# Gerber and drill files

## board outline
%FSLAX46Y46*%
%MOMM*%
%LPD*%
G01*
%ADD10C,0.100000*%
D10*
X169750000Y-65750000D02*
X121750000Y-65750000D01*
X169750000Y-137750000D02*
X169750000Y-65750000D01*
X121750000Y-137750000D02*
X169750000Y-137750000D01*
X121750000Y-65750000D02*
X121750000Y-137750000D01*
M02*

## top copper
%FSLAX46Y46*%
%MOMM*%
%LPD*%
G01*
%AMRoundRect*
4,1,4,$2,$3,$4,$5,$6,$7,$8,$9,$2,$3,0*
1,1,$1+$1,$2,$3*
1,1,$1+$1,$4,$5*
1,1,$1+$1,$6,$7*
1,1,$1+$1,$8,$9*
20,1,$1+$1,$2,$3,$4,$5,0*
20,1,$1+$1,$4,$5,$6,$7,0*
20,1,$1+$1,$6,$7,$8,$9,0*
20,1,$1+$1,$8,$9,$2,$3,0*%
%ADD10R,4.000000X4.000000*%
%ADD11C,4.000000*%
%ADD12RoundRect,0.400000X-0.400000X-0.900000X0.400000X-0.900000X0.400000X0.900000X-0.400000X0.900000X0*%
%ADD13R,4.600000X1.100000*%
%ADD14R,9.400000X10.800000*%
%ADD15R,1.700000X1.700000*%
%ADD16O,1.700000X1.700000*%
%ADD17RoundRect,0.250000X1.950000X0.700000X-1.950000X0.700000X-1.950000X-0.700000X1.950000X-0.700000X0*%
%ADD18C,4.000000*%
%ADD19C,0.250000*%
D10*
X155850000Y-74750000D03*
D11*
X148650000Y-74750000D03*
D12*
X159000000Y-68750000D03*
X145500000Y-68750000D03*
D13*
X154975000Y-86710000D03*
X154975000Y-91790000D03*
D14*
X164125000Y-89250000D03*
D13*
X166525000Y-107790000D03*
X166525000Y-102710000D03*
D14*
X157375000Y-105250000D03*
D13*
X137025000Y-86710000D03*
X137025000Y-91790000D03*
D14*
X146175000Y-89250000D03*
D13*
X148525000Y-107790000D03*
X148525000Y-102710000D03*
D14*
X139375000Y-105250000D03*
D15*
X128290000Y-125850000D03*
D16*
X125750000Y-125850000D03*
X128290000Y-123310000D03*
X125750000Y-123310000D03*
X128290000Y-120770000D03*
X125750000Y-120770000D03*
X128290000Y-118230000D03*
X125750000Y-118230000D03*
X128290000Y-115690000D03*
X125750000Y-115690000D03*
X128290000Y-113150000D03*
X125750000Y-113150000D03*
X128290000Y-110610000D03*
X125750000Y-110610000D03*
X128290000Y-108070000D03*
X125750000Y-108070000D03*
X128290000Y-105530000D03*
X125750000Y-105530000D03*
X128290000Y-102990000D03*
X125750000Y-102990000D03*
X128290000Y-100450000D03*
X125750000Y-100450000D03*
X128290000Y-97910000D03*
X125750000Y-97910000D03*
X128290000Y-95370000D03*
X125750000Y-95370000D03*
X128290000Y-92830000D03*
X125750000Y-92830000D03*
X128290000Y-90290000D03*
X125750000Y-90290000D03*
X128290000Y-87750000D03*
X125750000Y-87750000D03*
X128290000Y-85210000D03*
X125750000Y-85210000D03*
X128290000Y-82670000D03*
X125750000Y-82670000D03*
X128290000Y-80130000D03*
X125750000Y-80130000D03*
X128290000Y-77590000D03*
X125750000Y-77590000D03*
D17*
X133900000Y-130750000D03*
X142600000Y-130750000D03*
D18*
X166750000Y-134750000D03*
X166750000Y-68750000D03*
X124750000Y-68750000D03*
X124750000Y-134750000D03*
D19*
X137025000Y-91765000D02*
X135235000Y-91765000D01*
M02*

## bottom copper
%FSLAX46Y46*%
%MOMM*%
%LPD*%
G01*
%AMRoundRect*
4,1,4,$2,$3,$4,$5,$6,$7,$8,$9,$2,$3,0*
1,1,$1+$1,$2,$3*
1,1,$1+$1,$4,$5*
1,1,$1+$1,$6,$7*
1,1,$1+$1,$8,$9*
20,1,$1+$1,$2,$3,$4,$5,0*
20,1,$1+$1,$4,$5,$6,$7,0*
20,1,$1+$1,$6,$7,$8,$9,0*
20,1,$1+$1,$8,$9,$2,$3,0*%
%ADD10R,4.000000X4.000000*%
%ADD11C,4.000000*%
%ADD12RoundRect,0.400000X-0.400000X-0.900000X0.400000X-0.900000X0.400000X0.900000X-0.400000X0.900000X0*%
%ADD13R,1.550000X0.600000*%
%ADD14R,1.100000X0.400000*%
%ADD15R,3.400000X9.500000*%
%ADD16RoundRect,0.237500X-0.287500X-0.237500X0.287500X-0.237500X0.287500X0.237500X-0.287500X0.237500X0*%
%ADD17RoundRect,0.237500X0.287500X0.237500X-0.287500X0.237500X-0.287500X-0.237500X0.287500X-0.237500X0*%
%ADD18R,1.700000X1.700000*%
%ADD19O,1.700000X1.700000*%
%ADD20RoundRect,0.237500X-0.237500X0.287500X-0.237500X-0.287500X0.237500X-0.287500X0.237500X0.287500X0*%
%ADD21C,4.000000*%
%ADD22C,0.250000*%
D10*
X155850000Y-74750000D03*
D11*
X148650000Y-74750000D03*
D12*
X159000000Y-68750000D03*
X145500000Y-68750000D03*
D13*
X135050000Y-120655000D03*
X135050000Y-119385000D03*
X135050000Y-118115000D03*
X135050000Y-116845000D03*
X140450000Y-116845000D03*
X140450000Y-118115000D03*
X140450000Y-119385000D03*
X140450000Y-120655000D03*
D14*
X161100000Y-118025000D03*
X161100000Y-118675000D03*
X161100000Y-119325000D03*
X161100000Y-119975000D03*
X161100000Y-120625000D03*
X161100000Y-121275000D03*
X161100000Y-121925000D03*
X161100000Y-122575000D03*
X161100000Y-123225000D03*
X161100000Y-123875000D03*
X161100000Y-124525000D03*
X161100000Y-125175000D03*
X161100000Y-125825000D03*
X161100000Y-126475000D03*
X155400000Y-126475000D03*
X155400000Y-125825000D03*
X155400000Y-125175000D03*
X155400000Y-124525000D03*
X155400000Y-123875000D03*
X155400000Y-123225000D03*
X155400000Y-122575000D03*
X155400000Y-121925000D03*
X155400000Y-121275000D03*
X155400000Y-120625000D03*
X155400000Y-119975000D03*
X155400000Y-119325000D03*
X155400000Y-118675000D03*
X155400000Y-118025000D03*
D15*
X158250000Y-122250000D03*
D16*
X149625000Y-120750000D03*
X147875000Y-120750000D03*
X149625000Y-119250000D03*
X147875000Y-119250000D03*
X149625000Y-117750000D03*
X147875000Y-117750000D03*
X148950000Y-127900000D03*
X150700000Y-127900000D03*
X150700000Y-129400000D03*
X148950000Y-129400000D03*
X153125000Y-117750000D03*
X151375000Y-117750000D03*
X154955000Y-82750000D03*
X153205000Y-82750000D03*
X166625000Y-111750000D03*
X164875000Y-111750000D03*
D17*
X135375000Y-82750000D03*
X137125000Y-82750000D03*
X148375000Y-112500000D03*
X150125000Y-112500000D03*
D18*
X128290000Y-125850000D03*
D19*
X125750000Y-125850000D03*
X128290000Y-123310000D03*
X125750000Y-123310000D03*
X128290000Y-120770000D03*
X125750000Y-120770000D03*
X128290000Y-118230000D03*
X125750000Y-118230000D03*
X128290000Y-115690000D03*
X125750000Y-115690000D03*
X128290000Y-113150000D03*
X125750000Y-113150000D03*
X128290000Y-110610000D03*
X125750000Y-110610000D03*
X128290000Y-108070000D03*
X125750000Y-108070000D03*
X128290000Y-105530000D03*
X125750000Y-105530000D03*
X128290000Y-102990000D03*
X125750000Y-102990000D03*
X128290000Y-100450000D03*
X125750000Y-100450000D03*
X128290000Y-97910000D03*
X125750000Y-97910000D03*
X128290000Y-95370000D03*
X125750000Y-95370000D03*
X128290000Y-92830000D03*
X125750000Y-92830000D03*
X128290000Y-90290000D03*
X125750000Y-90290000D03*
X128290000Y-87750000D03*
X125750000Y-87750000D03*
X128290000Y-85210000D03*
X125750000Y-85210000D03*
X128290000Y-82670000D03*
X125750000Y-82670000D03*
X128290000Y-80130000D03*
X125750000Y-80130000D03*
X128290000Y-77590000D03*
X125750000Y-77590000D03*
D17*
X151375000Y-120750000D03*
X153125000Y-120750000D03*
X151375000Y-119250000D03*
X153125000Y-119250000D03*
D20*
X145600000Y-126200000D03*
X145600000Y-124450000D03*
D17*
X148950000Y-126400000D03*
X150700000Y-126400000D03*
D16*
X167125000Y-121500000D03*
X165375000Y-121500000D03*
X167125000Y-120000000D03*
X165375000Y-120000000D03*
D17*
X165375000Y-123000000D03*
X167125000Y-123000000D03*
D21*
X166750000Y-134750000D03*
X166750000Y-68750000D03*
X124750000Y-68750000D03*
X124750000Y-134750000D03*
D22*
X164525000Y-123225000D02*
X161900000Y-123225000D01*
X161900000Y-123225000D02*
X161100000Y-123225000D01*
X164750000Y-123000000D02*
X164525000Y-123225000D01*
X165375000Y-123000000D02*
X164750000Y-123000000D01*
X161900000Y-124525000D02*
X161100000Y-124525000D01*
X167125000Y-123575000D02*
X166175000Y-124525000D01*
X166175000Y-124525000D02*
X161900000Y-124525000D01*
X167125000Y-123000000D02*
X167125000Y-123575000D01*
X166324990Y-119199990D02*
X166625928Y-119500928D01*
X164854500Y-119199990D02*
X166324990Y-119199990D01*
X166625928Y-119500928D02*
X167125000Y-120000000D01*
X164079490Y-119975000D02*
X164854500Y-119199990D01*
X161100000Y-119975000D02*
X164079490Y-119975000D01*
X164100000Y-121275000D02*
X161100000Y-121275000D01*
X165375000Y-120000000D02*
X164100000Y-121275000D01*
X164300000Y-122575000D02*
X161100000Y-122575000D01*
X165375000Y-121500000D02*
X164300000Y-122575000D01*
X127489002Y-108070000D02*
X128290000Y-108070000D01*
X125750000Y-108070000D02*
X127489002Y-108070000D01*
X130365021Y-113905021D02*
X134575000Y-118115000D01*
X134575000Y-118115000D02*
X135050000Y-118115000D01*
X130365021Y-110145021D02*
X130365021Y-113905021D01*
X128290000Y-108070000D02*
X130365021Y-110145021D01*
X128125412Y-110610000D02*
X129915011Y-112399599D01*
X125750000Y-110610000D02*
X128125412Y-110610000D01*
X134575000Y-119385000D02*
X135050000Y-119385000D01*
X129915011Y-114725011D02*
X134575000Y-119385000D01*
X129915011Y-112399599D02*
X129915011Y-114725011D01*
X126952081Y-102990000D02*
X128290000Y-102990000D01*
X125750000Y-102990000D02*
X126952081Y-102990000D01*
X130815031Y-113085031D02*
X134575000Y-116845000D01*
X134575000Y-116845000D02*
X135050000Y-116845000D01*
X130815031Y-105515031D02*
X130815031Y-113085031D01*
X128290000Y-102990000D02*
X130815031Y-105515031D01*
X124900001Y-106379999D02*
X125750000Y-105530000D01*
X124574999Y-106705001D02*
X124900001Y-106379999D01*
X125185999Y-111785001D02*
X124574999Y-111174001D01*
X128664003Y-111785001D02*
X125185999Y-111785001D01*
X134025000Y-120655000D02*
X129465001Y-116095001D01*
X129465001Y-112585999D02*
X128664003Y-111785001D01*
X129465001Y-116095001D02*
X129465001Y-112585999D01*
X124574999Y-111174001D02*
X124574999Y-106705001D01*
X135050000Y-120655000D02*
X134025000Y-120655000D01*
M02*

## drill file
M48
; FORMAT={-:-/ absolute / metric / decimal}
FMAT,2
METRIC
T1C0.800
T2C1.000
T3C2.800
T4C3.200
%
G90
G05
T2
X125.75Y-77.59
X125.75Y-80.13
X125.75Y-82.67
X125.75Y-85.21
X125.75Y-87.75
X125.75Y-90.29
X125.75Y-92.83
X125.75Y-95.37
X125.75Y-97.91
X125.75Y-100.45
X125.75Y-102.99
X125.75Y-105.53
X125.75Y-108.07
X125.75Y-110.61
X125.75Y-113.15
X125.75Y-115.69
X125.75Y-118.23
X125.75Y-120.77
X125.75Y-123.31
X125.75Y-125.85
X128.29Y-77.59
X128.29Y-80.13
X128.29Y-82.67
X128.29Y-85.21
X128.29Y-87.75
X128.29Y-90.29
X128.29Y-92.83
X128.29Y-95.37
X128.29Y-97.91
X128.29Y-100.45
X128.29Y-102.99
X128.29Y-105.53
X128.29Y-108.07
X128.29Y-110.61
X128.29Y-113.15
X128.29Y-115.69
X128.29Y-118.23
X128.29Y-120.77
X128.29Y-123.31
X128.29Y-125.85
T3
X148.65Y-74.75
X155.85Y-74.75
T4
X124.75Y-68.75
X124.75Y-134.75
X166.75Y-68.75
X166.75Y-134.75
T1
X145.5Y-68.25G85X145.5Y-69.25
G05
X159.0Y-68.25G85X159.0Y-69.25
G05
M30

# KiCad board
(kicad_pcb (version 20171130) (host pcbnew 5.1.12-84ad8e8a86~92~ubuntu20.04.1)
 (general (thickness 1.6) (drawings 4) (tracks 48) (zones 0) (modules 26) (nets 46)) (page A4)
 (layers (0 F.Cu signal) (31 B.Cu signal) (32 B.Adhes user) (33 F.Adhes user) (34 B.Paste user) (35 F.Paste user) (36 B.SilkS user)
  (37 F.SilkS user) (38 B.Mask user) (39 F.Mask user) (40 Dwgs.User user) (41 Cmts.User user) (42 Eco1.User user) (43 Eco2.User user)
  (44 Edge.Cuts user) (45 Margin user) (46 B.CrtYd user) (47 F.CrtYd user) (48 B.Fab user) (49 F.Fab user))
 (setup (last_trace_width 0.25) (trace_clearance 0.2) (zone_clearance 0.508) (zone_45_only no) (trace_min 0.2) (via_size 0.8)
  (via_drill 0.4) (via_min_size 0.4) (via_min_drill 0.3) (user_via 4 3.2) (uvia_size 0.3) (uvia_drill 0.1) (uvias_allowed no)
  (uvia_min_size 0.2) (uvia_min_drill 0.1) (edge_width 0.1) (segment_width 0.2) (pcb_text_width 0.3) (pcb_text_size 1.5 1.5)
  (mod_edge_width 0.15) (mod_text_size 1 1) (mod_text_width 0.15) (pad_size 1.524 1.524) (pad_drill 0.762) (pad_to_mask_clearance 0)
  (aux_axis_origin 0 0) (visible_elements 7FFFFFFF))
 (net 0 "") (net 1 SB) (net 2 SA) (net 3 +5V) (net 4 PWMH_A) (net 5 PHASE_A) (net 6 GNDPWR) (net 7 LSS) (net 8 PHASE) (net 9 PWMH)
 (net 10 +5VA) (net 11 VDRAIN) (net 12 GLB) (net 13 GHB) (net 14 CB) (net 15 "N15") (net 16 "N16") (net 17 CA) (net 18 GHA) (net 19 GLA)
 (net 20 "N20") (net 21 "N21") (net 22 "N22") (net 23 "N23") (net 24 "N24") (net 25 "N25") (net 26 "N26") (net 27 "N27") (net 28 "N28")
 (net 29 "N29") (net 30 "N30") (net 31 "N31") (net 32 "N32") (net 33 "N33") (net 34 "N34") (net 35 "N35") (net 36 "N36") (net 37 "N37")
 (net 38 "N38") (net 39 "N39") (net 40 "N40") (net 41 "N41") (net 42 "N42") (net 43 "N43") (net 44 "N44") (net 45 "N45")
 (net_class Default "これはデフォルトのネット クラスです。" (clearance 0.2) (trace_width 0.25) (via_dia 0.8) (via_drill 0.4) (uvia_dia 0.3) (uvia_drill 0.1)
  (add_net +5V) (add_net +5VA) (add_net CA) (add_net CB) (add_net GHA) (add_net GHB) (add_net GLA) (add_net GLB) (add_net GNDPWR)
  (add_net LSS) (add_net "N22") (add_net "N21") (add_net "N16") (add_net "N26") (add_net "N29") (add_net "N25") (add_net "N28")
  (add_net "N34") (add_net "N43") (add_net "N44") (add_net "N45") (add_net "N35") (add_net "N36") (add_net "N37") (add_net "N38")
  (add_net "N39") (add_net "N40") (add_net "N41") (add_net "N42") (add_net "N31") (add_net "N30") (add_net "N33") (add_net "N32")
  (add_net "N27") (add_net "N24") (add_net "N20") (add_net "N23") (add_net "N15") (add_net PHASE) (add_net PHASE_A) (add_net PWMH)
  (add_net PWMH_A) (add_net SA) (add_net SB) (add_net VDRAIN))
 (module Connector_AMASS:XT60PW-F (layer F.Cu) (at 152.25 74.75)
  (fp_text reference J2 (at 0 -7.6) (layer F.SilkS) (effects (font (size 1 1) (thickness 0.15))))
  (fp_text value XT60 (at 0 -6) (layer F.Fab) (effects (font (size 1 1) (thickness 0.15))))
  (pad 1 thru_hole rect (at 3.6 0) (size 4 4) (drill 2.8) (layers *.Cu *.Mask) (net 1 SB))
  (pad 2 thru_hole circle (at -3.6 0) (size 4 4) (drill 2.8) (layers *.Cu *.Mask) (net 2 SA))
  (pad 2 thru_hole roundrect (at 6.75 -6) (size 1.6 2.6) (drill oval 0.8 1.8) (layers *.Cu *.Mask) (roundrect_rratio 0.25) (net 2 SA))
  (pad 1 thru_hole roundrect (at -6.75 -6) (size 1.6 2.6) (drill oval 0.8 1.8) (layers *.Cu *.Mask) (roundrect_rratio 0.25) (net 1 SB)))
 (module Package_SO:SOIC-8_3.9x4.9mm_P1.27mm (layer B.Cu) (at 137.75 118.75)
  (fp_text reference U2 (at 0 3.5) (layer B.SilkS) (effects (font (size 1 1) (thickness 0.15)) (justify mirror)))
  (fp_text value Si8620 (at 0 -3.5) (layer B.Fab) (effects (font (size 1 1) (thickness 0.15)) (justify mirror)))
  (pad 1 smd rect (at -2.7 1.905) (size 1.55 0.6) (layers B.Cu B.Paste B.Mask) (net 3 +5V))
  (pad 2 smd rect (at -2.7 0.635) (size 1.55 0.6) (layers B.Cu B.Paste B.Mask) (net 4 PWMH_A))
  (pad 3 smd rect (at -2.7 -0.635) (size 1.55 0.6) (layers B.Cu B.Paste B.Mask) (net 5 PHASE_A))
  (pad 4 smd rect (at -2.7 -1.905) (size 1.55 0.6) (layers B.Cu B.Paste B.Mask) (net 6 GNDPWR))
  (pad 5 smd rect (at 2.7 -1.905) (size 1.55 0.6) (layers B.Cu B.Paste B.Mask) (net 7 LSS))
  (pad 6 smd rect (at 2.7 -0.635) (size 1.55 0.6) (layers B.Cu B.Paste B.Mask) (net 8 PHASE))
  (pad 7 smd rect (at 2.7 0.635) (size 1.55 0.6) (layers B.Cu B.Paste B.Mask) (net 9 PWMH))
  (pad 8 smd rect (at 2.7 1.905) (size 1.55 0.6) (layers B.Cu B.Paste B.Mask) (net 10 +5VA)))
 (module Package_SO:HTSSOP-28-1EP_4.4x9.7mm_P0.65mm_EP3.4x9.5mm (layer B.Cu) (at 158.25 122.25 180)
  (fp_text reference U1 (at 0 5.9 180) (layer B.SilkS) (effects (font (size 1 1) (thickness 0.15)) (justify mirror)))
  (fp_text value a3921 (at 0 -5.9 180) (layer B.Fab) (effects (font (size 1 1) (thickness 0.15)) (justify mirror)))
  (pad 1 smd rect (at -2.85 4.225 180) (size 1.1 0.4) (layers B.Cu B.Paste B.Mask) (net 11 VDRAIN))
  (pad 2 smd rect (at -2.85 3.575 180) (size 1.1 0.4) (layers B.Cu B.Paste B.Mask) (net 7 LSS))
  (pad 3 smd rect (at -2.85 2.925 180) (size 1.1 0.4) (layers B.Cu B.Paste B.Mask) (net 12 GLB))
  (pad 4 smd rect (at -2.85 2.275 180) (size 1.1 0.4) (layers B.Cu B.Paste B.Mask) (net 1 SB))
  (pad 5 smd rect (at -2.85 1.625 180) (size 1.1 0.4) (layers B.Cu B.Paste B.Mask) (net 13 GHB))
  (pad 6 smd rect (at -2.85 0.975 180) (size 1.1 0.4) (layers B.Cu B.Paste B.Mask) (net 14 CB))
  (pad 7 smd rect (at -2.85 0.325 180) (size 1.1 0.4) (layers B.Cu B.Paste B.Mask) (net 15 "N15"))
  (pad 8 smd rect (at -2.85 -0.325 180) (size 1.1 0.4) (layers B.Cu B.Paste B.Mask) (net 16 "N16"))
  (pad 9 smd rect (at -2.85 -0.975 180) (size 1.1 0.4) (layers B.Cu B.Paste B.Mask) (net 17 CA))
  (pad 10 smd rect (at -2.85 -1.625 180) (size 1.1 0.4) (layers B.Cu B.Paste B.Mask) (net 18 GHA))
  (pad 11 smd rect (at -2.85 -2.275 180) (size 1.1 0.4) (layers B.Cu B.Paste B.Mask) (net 2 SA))
  (pad 12 smd rect (at -2.85 -2.925 180) (size 1.1 0.4) (layers B.Cu B.Paste B.Mask) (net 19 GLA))
  (pad 13 smd rect (at -2.85 -3.575 180) (size 1.1 0.4) (layers B.Cu B.Paste B.Mask) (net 11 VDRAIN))
  (pad 14 smd rect (at -2.85 -4.225 180) (size 1.1 0.4) (layers B.Cu B.Paste B.Mask) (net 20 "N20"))
  (pad 15 smd rect (at 2.85 -4.225 180) (size 1.1 0.4) (layers B.Cu B.Paste B.Mask) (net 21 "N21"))
  (pad 16 smd rect (at 2.85 -3.575 180) (size 1.1 0.4) (layers B.Cu B.Paste B.Mask) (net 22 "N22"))
  (pad 17 smd rect (at 2.85 -2.925 180) (size 1.1 0.4) (layers B.Cu B.Paste B.Mask) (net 7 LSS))
  (pad 18 smd rect (at 2.85 -2.275 180) (size 1.1 0.4) (layers B.Cu B.Paste B.Mask) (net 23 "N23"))
  (pad 19 smd rect (at 2.85 -1.625 180) (size 1.1 0.4) (layers B.Cu B.Paste B.Mask) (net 8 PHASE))
  (pad 20 smd rect (at 2.85 -0.975 180) (size 1.1 0.4) (layers B.Cu B.Paste B.Mask) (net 10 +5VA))
  (pad 21 smd rect (at 2.85 -0.325 180) (size 1.1 0.4) (layers B.Cu B.Paste B.Mask) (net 10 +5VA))
  (pad 22 smd rect (at 2.85 0.325 180) (size 1.1 0.4) (layers B.Cu B.Paste B.Mask) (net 10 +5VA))
  (pad 23 smd rect (at 2.85 0.975 180) (size 1.1 0.4) (layers B.Cu B.Paste B.Mask) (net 9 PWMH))
  (pad 24 smd rect (at 2.85 1.625 180) (size 1.1 0.4) (layers B.Cu B.Paste B.Mask) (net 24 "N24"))
  (pad 25 smd rect (at 2.85 2.275 180) (size 1.1 0.4) (layers B.Cu B.Paste B.Mask) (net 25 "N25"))
  (pad 26 smd rect (at 2.85 2.925 180) (size 1.1 0.4) (layers B.Cu B.Paste B.Mask) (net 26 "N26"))
  (pad 27 smd rect (at 2.85 3.575 180) (size 1.1 0.4) (layers B.Cu B.Paste B.Mask) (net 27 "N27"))
  (pad 28 smd rect (at 2.85 4.225 180) (size 1.1 0.4) (layers B.Cu B.Paste B.Mask) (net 10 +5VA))
  (pad 29 smd rect (at 0 0 180) (size 3.4 9.5) (layers B.Cu B.Mask))
  (pad "" smd rect (at -0.85 3.8 180) (size 1.4 1.6) (layers B.Paste))
  (pad "" smd rect (at 0.85 3.8 180) (size 1.4 1.6) (layers B.Paste))
  (pad "" smd rect (at 0.85 1.9 180) (size 1.4 1.6) (layers B.Paste))
  (pad "" smd rect (at -0.85 1.9 180) (size 1.4 1.6) (layers B.Paste))
  (pad "" smd rect (at 0.85 0 180) (size 1.4 1.6) (layers B.Paste))
  (pad "" smd rect (at -0.85 0 180) (size 1.4 1.6) (layers B.Paste))
  (pad "" smd rect (at 0.85 -1.9 180) (size 1.4 1.6) (layers B.Paste))
  (pad "" smd rect (at -0.85 -1.9 180) (size 1.4 1.6) (layers B.Paste))
  (pad "" smd rect (at 0.85 -3.8 180) (size 1.4 1.6) (layers B.Paste))
  (pad "" smd rect (at -0.85 -3.8 180) (size 1.4 1.6) (layers B.Paste)))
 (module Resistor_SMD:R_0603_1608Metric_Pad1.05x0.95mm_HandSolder (layer B.Cu) (at 148.75 120.75)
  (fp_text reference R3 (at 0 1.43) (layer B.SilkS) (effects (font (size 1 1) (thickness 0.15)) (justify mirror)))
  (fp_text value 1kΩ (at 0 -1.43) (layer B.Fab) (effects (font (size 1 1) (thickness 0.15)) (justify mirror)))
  (pad 2 smd roundrect (at 0.875 0) (size 1.05 0.95) (layers B.Cu B.Paste B.Mask) (roundrect_rratio 0.25) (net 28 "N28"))
  (pad 1 smd roundrect (at -0.875 0) (size 1.05 0.95) (layers B.Cu B.Paste B.Mask) (roundrect_rratio 0.25) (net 10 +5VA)))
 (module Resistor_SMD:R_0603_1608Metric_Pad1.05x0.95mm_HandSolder (layer B.Cu) (at 148.75 119.25)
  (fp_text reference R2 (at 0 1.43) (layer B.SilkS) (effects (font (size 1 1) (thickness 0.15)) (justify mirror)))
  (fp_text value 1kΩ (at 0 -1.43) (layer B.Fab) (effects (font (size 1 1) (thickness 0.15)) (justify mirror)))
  (pad 2 smd roundrect (at 0.875 0) (size 1.05 0.95) (layers B.Cu B.Paste B.Mask) (roundrect_rratio 0.25) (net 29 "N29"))
  (pad 1 smd roundrect (at -0.875 0) (size 1.05 0.95) (layers B.Cu B.Paste B.Mask) (roundrect_rratio 0.25) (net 10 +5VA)))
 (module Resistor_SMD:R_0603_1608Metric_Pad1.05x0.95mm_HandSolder (layer B.Cu) (at 148.75 117.75)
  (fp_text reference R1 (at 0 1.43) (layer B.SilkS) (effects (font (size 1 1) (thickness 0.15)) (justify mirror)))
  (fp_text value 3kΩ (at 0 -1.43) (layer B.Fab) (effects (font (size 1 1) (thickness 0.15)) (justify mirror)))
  (pad 2 smd roundrect (at 0.875 0) (size 1.05 0.95) (layers B.Cu B.Paste B.Mask) (roundrect_rratio 0.25) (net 27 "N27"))
  (pad 1 smd roundrect (at -0.875 0) (size 1.05 0.95) (layers B.Cu B.Paste B.Mask) (roundrect_rratio 0.25) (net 7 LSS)))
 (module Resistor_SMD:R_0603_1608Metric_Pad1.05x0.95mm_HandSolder (layer B.Cu) (at 149.825 127.9)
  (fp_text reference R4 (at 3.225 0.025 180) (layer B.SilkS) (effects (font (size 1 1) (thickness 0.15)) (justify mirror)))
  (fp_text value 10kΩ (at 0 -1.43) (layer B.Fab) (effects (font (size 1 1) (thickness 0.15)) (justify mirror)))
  (pad 1 smd roundrect (at -0.875 0) (size 1.05 0.95) (layers B.Cu B.Paste B.Mask) (roundrect_rratio 0.25) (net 8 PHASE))
  (pad 2 smd roundrect (at 0.875 0) (size 1.05 0.95) (layers B.Cu B.Paste B.Mask) (roundrect_rratio 0.25) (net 7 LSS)))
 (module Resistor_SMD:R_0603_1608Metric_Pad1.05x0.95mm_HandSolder (layer B.Cu) (at 149.825 129.4)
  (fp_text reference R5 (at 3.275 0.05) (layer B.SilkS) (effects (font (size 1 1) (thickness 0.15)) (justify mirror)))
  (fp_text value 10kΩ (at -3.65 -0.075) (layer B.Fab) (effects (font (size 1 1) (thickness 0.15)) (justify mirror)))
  (pad 2 smd roundrect (at 0.875 0) (size 1.05 0.95) (layers B.Cu B.Paste B.Mask) (roundrect_rratio 0.25) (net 7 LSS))
  (pad 1 smd roundrect (at -0.875 0) (size 1.05 0.95) (layers B.Cu B.Paste B.Mask) (roundrect_rratio 0.25) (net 9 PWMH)))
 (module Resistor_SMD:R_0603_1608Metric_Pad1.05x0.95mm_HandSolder (layer B.Cu) (at 152.25 117.75)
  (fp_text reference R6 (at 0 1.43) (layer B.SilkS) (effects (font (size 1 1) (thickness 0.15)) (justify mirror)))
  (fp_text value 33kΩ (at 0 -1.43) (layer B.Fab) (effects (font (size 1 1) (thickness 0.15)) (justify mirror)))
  (pad 2 smd roundrect (at 0.875 0) (size 1.05 0.95) (layers B.Cu B.Paste B.Mask) (roundrect_rratio 0.25) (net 24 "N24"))
  (pad 1 smd roundrect (at -0.875 0) (size 1.05 0.95) (layers B.Cu B.Paste B.Mask) (roundrect_rratio 0.25) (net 11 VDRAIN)))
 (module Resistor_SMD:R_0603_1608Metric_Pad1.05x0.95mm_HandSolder (layer B.Cu) (at 154.08 82.75)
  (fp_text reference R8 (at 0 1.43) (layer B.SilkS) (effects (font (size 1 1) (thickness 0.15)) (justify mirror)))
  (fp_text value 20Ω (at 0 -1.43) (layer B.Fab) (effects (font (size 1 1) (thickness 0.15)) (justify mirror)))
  (pad 2 smd roundrect (at 0.875 0) (size 1.05 0.95) (layers B.Cu B.Paste B.Mask) (roundrect_rratio 0.25) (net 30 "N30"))
  (pad 1 smd roundrect (at -0.875 0) (size 1.05 0.95) (layers B.Cu B.Paste B.Mask) (roundrect_rratio 0.25) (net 12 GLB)))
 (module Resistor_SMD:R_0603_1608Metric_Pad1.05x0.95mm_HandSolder (layer B.Cu) (at 165.75 111.75)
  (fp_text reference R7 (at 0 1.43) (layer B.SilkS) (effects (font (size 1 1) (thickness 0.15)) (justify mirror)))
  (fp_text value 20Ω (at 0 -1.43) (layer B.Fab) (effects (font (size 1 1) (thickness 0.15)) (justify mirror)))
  (pad 2 smd roundrect (at 0.875 0) (size 1.05 0.95) (layers B.Cu B.Paste B.Mask) (roundrect_rratio 0.25) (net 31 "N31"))
  (pad 1 smd roundrect (at -0.875 0) (size 1.05 0.95) (layers B.Cu B.Paste B.Mask) (roundrect_rratio 0.25) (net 13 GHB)))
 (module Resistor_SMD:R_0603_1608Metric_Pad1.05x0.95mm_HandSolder (layer B.Cu) (at 136.25 82.75 180)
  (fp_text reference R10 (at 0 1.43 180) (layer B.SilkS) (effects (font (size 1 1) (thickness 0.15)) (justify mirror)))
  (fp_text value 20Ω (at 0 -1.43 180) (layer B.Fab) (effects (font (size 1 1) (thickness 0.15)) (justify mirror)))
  (pad 2 smd roundrect (at 0.875 0 180) (size 1.05 0.95) (layers B.Cu B.Paste B.Mask) (roundrect_rratio 0.25) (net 19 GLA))
  (pad 1 smd roundrect (at -0.875 0 180) (size 1.05 0.95) (layers B.Cu B.Paste B.Mask) (roundrect_rratio 0.25) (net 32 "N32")))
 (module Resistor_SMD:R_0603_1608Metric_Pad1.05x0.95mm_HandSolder (layer B.Cu) (at 149.25 112.5 180)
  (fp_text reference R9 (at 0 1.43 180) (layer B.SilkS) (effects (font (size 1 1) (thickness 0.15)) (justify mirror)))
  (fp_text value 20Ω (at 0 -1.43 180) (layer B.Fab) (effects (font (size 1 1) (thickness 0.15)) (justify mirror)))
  (pad 2 smd roundrect (at 0.875 0 180) (size 1.05 0.95) (layers B.Cu B.Paste B.Mask) (roundrect_rratio 0.25) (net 18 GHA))
  (pad 1 smd roundrect (at -0.875 0 180) (size 1.05 0.95) (layers B.Cu B.Paste B.Mask) (roundrect_rratio 0.25) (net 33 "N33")))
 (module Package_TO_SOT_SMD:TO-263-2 (layer F.Cu) (at 160.75 89.25)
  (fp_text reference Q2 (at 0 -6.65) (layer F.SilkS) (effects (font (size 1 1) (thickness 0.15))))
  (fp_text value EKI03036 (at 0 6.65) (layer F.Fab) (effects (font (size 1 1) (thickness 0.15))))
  (pad 1 smd rect (at -5.775 -2.54) (size 4.6 1.1) (layers F.Cu F.Paste F.Mask) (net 30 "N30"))
  (pad 3 smd rect (at -5.775 2.54) (size 4.6 1.1) (layers F.Cu F.Paste F.Mask) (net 7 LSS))
  (pad 2 smd rect (at 3.375 0) (size 9.4 10.8) (layers F.Cu F.Mask) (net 1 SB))
  (pad "" smd rect (at 5.8 2.775) (size 4.55 5.25) (layers F.Paste))
  (pad "" smd rect (at 0.95 -2.775) (size 4.55 5.25) (layers F.Paste))
  (pad "" smd rect (at 5.8 -2.775) (size 4.55 5.25) (layers F.Paste))
  (pad "" smd rect (at 0.95 2.775) (size 4.55 5.25) (layers F.Paste)))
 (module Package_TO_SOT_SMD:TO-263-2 (layer F.Cu) (at 160.75 105.25 180)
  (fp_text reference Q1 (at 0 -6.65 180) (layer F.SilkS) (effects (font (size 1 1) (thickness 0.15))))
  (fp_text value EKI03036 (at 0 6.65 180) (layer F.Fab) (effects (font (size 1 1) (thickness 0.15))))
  (pad 1 smd rect (at -5.775 -2.54 180) (size 4.6 1.1) (layers F.Cu F.Paste F.Mask) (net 31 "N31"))
  (pad 3 smd rect (at -5.775 2.54 180) (size 4.6 1.1) (layers F.Cu F.Paste F.Mask) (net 1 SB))
  (pad 2 smd rect (at 3.375 0 180) (size 9.4 10.8) (layers F.Cu F.Mask) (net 11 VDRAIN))
  (pad "" smd rect (at 5.8 2.775 180) (size 4.55 5.25) (layers F.Paste))
  (pad "" smd rect (at 0.95 -2.775 180) (size 4.55 5.25) (layers F.Paste))
  (pad "" smd rect (at 5.8 -2.775 180) (size 4.55 5.25) (layers F.Paste))
  (pad "" smd rect (at 0.95 2.775 180) (size 4.55 5.25) (layers F.Paste)))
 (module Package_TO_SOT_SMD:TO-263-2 (layer F.Cu) (at 142.8 89.25)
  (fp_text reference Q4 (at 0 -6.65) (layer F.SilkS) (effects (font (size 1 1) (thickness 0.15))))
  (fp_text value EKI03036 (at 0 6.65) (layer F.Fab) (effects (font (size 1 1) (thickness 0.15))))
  (pad 1 smd rect (at -5.775 -2.54) (size 4.6 1.1) (layers F.Cu F.Paste F.Mask) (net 32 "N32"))
  (pad 3 smd rect (at -5.775 2.54) (size 4.6 1.1) (layers F.Cu F.Paste F.Mask) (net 7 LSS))
  (pad 2 smd rect (at 3.375 0) (size 9.4 10.8) (layers F.Cu F.Mask) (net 2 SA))
  (pad "" smd rect (at 5.8 2.775) (size 4.55 5.25) (layers F.Paste))
  (pad "" smd rect (at 0.95 -2.775) (size 4.55 5.25) (layers F.Paste))
  (pad "" smd rect (at 5.8 -2.775) (size 4.55 5.25) (layers F.Paste))
  (pad "" smd rect (at 0.95 2.775) (size 4.55 5.25) (layers F.Paste)))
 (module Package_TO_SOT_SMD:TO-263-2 (layer F.Cu) (at 142.75 105.25 180)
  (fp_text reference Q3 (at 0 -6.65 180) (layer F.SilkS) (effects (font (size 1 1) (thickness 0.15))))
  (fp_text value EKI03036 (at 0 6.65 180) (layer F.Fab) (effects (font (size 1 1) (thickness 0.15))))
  (pad 1 smd rect (at -5.775 -2.54 180) (size 4.6 1.1) (layers F.Cu F.Paste F.Mask) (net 33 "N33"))
  (pad 3 smd rect (at -5.775 2.54 180) (size 4.6 1.1) (layers F.Cu F.Paste F.Mask) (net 2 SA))
  (pad 2 smd rect (at 3.375 0 180) (size 9.4 10.8) (layers F.Cu F.Mask) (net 11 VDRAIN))
  (pad "" smd rect (at 5.8 2.775 180) (size 4.55 5.25) (layers F.Paste))
  (pad "" smd rect (at 0.95 -2.775 180) (size 4.55 5.25) (layers F.Paste))
  (pad "" smd rect (at 5.8 -2.775 180) (size 4.55 5.25) (layers F.Paste))
  (pad "" smd rect (at 0.95 2.775 180) (size 4.55 5.25) (layers F.Paste)))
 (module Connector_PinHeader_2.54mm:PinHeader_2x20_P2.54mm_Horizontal (layer F.Cu) (at 128.29 125.85 180)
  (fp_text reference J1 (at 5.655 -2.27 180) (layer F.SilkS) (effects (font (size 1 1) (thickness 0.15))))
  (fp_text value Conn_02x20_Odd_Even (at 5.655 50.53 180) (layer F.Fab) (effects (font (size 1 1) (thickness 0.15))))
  (pad 1 thru_hole rect (at 0 0 180) (size 1.7 1.7) (drill 1) (layers *.Cu *.Mask) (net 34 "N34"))
  (pad 2 thru_hole oval (at 2.54 0 180) (size 1.7 1.7) (drill 1) (layers *.Cu *.Mask) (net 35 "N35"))
  (pad 3 thru_hole oval (at 0 2.54 180) (size 1.7 1.7) (drill 1) (layers *.Cu *.Mask) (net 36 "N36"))
  (pad 4 thru_hole oval (at 2.54 2.54 180) (size 1.7 1.7) (drill 1) (layers *.Cu *.Mask) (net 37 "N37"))
  (pad 5 thru_hole oval (at 0 5.08 180) (size 1.7 1.7) (drill 1) (layers *.Cu *.Mask) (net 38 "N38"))
  (pad 6 thru_hole oval (at 2.54 5.08 180) (size 1.7 1.7) (drill 1) (layers *.Cu *.Mask) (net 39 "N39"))
  (pad 7 thru_hole oval (at 0 7.62 180) (size 1.7 1.7) (drill 1) (layers *.Cu *.Mask) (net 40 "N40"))
  (pad 8 thru_hole oval (at 2.54 7.62 180) (size 1.7 1.7) (drill 1) (layers *.Cu *.Mask) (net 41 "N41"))
  (pad 9 thru_hole oval (at 0 10.16 180) (size 1.7 1.7) (drill 1) (layers *.Cu *.Mask) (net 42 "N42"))
  (pad 10 thru_hole oval (at 2.54 10.16 180) (size 1.7 1.7) (drill 1) (layers *.Cu *.Mask) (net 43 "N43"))
  (pad 11 thru_hole oval (at 0 12.7 180) (size 1.7 1.7) (drill 1) (layers *.Cu *.Mask) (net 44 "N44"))
  (pad 12 thru_hole oval (at 2.54 12.7 180) (size 1.7 1.7) (drill 1) (layers *.Cu *.Mask) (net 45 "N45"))
  (pad 13 thru_hole oval (at 0 15.24 180) (size 1.7 1.7) (drill 1) (layers *.Cu *.Mask) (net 4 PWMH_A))
  (pad 14 thru_hole oval (at 2.54 15.24 180) (size 1.7 1.7) (drill 1) (layers *.Cu *.Mask) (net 4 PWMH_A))
  (pad 15 thru_hole oval (at 0 17.78 180) (size 1.7 1.7) (drill 1) (layers *.Cu *.Mask) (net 5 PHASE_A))
  (pad 16 thru_hole oval (at 2.54 17.78 180) (size 1.7 1.7) (drill 1) (layers *.Cu *.Mask) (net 5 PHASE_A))
  (pad 17 thru_hole oval (at 0 20.32 180) (size 1.7 1.7) (drill 1) (layers *.Cu *.Mask) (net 3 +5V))
  (pad 18 thru_hole oval (at 2.54 20.32 180) (size 1.7 1.7) (drill 1) (layers *.Cu *.Mask) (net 3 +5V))
  (pad 19 thru_hole oval (at 0 22.86 180) (size 1.7 1.7) (drill 1) (layers *.Cu *.Mask) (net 6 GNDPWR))
  (pad 20 thru_hole oval (at 2.54 22.86 180) (size 1.7 1.7) (drill 1) (layers *.Cu *.Mask) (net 6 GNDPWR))
  (pad 21 thru_hole oval (at 0 25.4 180) (size 1.7 1.7) (drill 1) (layers *.Cu *.Mask) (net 11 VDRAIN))
  (pad 22 thru_hole oval (at 2.54 25.4 180) (size 1.7 1.7) (drill 1) (layers *.Cu *.Mask) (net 11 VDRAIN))
  (pad 23 thru_hole oval (at 0 27.94 180) (size 1.7 1.7) (drill 1) (layers *.Cu *.Mask) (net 11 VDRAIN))
  (pad 24 thru_hole oval (at 2.54 27.94 180) (size 1.7 1.7) (drill 1) (layers *.Cu *.Mask) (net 11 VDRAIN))
  (pad 25 thru_hole oval (at 0 30.48 180) (size 1.7 1.7) (drill 1) (layers *.Cu *.Mask) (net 11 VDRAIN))
  (pad 26 thru_hole oval (at 2.54 30.48 180) (size 1.7 1.7) (drill 1) (layers *.Cu *.Mask) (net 11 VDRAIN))
  (pad 27 thru_hole oval (at 0 33.02 180) (size 1.7 1.7) (drill 1) (layers *.Cu *.Mask) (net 11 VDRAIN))
  (pad 28 thru_hole oval (at 2.54 33.02 180) (size 1.7 1.7) (drill 1) (layers *.Cu *.Mask) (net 11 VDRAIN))
  (pad 29 thru_hole oval (at 0 35.56 180) (size 1.7 1.7) (drill 1) (layers *.Cu *.Mask) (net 11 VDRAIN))
  (pad 30 thru_hole oval (at 2.54 35.56 180) (size 1.7 1.7) (drill 1) (layers *.Cu *.Mask) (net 11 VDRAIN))
  (pad 31 thru_hole oval (at 0 38.1 180) (size 1.7 1.7) (drill 1) (layers *.Cu *.Mask) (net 7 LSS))
  (pad 32 thru_hole oval (at 2.54 38.1 180) (size 1.7 1.7) (drill 1) (layers *.Cu *.Mask) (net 7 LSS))
  (pad 33 thru_hole oval (at 0 40.64 180) (size 1.7 1.7) (drill 1) (layers *.Cu *.Mask) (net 7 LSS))
  (pad 34 thru_hole oval (at 2.54 40.64 180) (size 1.7 1.7) (drill 1) (layers *.Cu *.Mask) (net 7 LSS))
  (pad 35 thru_hole oval (at 0 43.18 180) (size 1.7 1.7) (drill 1) (layers *.Cu *.Mask) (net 7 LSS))
  (pad 36 thru_hole oval (at 2.54 43.18 180) (size 1.7 1.7) (drill 1) (layers *.Cu *.Mask) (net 7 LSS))
  (pad 37 thru_hole oval (at 0 45.72 180) (size 1.7 1.7) (drill 1) (layers *.Cu *.Mask) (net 7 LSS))
  (pad 38 thru_hole oval (at 2.54 45.72 180) (size 1.7 1.7) (drill 1) (layers *.Cu *.Mask) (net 7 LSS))
  (pad 39 thru_hole oval (at 0 48.26 180) (size 1.7 1.7) (drill 1) (layers *.Cu *.Mask) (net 7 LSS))
  (pad 40 thru_hole oval (at 2.54 48.26 180) (size 1.7 1.7) (drill 1) (layers *.Cu *.Mask) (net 7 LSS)))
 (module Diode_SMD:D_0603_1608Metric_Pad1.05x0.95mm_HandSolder (layer B.Cu) (at 152.25 120.75 180)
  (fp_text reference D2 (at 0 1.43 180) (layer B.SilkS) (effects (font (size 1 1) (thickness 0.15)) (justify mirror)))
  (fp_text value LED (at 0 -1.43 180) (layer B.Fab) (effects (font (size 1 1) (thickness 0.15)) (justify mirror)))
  (pad 2 smd roundrect (at 0.875 0 180) (size 1.05 0.95) (layers B.Cu B.Paste B.Mask) (roundrect_rratio 0.25) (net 28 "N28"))
  (pad 1 smd roundrect (at -0.875 0 180) (size 1.05 0.95) (layers B.Cu B.Paste B.Mask) (roundrect_rratio 0.25) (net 25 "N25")))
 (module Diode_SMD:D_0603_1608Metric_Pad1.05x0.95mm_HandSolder (layer B.Cu) (at 152.25 119.25 180)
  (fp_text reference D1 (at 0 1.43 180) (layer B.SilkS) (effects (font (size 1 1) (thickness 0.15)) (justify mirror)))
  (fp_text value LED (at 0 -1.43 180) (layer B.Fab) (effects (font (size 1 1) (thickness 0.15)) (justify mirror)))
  (pad 2 smd roundrect (at 0.875 0 180) (size 1.05 0.95) (layers B.Cu B.Paste B.Mask) (roundrect_rratio 0.25) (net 29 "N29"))
  (pad 1 smd roundrect (at -0.875 0 180) (size 1.05 0.95) (layers B.Cu B.Paste B.Mask) (roundrect_rratio 0.25) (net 26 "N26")))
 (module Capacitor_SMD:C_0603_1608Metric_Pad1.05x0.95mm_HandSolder (layer B.Cu) (at 145.6 125.325 270)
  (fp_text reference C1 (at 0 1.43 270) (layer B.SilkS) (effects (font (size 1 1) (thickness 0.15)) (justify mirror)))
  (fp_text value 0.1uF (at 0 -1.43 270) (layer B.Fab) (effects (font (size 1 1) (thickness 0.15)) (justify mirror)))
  (pad 2 smd roundrect (at 0.875 0 270) (size 1.05 0.95) (layers B.Cu B.Paste B.Mask) (roundrect_rratio 0.25) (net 7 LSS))
  (pad 1 smd roundrect (at -0.875 0 270) (size 1.05 0.95) (layers B.Cu B.Paste B.Mask) (roundrect_rratio 0.25) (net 10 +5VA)))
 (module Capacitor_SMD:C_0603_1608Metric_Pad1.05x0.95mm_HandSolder (layer B.Cu) (at 149.825 126.4 180)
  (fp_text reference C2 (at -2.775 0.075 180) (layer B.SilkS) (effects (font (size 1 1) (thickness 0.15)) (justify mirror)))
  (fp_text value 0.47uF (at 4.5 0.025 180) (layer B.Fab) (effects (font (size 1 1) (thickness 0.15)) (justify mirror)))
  (pad 2 smd roundrect (at 0.875 0 180) (size 1.05 0.95) (layers B.Cu B.Paste B.Mask) (roundrect_rratio 0.25) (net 21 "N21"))
  (pad 1 smd roundrect (at -0.875 0 180) (size 1.05 0.95) (layers B.Cu B.Paste B.Mask) (roundrect_rratio 0.25) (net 22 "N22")))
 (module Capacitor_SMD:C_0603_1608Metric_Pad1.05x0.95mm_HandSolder (layer B.Cu) (at 166.25 121.5)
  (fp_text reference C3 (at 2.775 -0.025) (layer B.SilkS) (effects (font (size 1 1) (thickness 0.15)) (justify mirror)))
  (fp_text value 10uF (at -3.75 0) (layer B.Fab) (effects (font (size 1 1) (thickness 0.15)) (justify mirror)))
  (pad 2 smd roundrect (at 0.875 0) (size 1.05 0.95) (layers B.Cu B.Paste B.Mask) (roundrect_rratio 0.25) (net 7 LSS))
  (pad 1 smd roundrect (at -0.875 0) (size 1.05 0.95) (layers B.Cu B.Paste B.Mask) (roundrect_rratio 0.25) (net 16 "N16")))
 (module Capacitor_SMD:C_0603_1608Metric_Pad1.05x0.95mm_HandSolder (layer B.Cu) (at 166.25 120)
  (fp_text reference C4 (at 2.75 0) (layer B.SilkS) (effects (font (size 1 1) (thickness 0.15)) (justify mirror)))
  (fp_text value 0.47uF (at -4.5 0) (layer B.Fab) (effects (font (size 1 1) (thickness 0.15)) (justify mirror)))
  (pad 2 smd roundrect (at 0.875 0) (size 1.05 0.95) (layers B.Cu B.Paste B.Mask) (roundrect_rratio 0.25) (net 1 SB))
  (pad 1 smd roundrect (at -0.875 0) (size 1.05 0.95) (layers B.Cu B.Paste B.Mask) (roundrect_rratio 0.25) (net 14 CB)))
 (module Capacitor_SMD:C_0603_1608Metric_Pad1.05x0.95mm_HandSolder (layer B.Cu) (at 166.25 123 180)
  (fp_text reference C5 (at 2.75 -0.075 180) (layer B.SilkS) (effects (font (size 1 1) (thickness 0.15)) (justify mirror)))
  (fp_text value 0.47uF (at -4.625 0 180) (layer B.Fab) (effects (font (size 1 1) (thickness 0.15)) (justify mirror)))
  (pad 2 smd roundrect (at 0.875 0 180) (size 1.05 0.95) (layers B.Cu B.Paste B.Mask) (roundrect_rratio 0.25) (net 17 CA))
  (pad 1 smd roundrect (at -0.875 0 180) (size 1.05 0.95) (layers B.Cu B.Paste B.Mask) (roundrect_rratio 0.25) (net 2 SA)))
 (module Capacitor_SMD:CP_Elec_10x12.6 (layer F.Cu) (at 138.25 130.75 180)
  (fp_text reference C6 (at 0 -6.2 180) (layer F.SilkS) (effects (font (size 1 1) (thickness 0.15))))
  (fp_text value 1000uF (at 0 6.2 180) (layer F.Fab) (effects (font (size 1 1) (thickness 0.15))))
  (pad 2 smd roundrect (at 4.35 0 180) (size 4.4 1.9) (layers F.Cu F.Paste F.Mask) (roundrect_rratio 0.131579) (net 7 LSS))
  (pad 1 smd roundrect (at -4.35 0 180) (size 4.4 1.9) (layers F.Cu F.Paste F.Mask) (roundrect_rratio 0.131579) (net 11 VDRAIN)))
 (gr_line (start 169.75 65.75) (end 121.75 65.75) (layer Edge.Cuts) (width 0.1))
 (gr_line (start 169.75 137.75) (end 169.75 65.75) (layer Edge.Cuts) (width 0.1))
 (gr_line (start 121.75 137.75) (end 169.75 137.75) (layer Edge.Cuts) (width 0.1))
 (gr_line (start 121.75 65.75) (end 121.75 137.75) (layer Edge.Cuts) (width 0.1))
 (via (at 166.75 134.75) (size 4) (drill 3.2) (layers F.Cu B.Cu) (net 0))
 (via (at 166.75 68.75) (size 4) (drill 3.2) (layers F.Cu B.Cu) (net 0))
 (via (at 124.75 68.75) (size 4) (drill 3.2) (layers F.Cu B.Cu) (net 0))
 (via (at 124.75 134.75) (size 4) (drill 3.2) (layers F.Cu B.Cu) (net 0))
 (segment (start 137.025 91.765) (end 135.235 91.765) (width 0.25) (layer F.Cu) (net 7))
 (segment (start 164.525 123.225) (end 161.9 123.225) (width 0.25) (layer B.Cu) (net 17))
 (segment (start 161.9 123.225) (end 161.1 123.225) (width 0.25) (layer B.Cu) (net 17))
 (segment (start 164.75 123) (end 164.525 123.225) (width 0.25) (layer B.Cu) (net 17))
 (segment (start 165.375 123) (end 164.75 123) (width 0.25) (layer B.Cu) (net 17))
 (segment (start 161.9 124.525) (end 161.1 124.525) (width 0.25) (layer B.Cu) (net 2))
 (segment (start 167.125 123.575) (end 166.175 124.525) (width 0.25) (layer B.Cu) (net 2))
 (segment (start 166.175 124.525) (end 161.9 124.525) (width 0.25) (layer B.Cu) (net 2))
 (segment (start 167.125 123) (end 167.125 123.575) (width 0.25) (layer B.Cu) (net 2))
 (segment (start 166.32499 119.19999) (end 166.625928 119.500928) (width 0.25) (layer B.Cu) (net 1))
 (segment (start 164.8545 119.19999) (end 166.32499 119.19999) (width 0.25) (layer B.Cu) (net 1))
 (segment (start 166.625928 119.500928) (end 167.125 120) (width 0.25) (layer B.Cu) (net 1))
 (segment (start 164.07949 119.975) (end 164.8545 119.19999) (width 0.25) (layer B.Cu) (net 1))
 (segment (start 161.1 119.975) (end 164.07949 119.975) (width 0.25) (layer B.Cu) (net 1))
 (segment (start 164.1 121.275) (end 161.1 121.275) (width 0.25) (layer B.Cu) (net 14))
 (segment (start 165.375 120) (end 164.1 121.275) (width 0.25) (layer B.Cu) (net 14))
 (segment (start 164.3 122.575) (end 161.1 122.575) (width 0.25) (layer B.Cu) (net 16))
 (segment (start 165.375 121.5) (end 164.3 122.575) (width 0.25) (layer B.Cu) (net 16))
 (segment (start 127.489002 108.07) (end 128.29 108.07) (width 0.25) (layer B.Cu) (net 5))
 (segment (start 125.75 108.07) (end 127.489002 108.07) (width 0.25) (layer B.Cu) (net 5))
 (segment (start 130.365021 113.905021) (end 134.575 118.115) (width 0.25) (layer B.Cu) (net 5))
 (segment (start 134.575 118.115) (end 135.05 118.115) (width 0.25) (layer B.Cu) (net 5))
 (segment (start 130.365021 110.145021) (end 130.365021 113.905021) (width 0.25) (layer B.Cu) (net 5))
 (segment (start 128.29 108.07) (end 130.365021 110.145021) (width 0.25) (layer B.Cu) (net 5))
 (segment (start 128.125412 110.61) (end 129.915011 112.399599) (width 0.25) (layer B.Cu) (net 4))
 (segment (start 125.75 110.61) (end 128.125412 110.61) (width 0.25) (layer B.Cu) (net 4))
 (segment (start 134.575 119.385) (end 135.05 119.385) (width 0.25) (layer B.Cu) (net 4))
 (segment (start 129.915011 114.725011) (end 134.575 119.385) (width 0.25) (layer B.Cu) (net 4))
 (segment (start 129.915011 112.399599) (end 129.915011 114.725011) (width 0.25) (layer B.Cu) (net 4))
 (segment (start 126.952081 102.99) (end 128.29 102.99) (width 0.25) (layer B.Cu) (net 6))
 (segment (start 125.75 102.99) (end 126.952081 102.99) (width 0.25) (layer B.Cu) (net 6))
 (segment (start 130.815031 113.085031) (end 134.575 116.845) (width 0.25) (layer B.Cu) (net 6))
 (segment (start 134.575 116.845) (end 135.05 116.845) (width 0.25) (layer B.Cu) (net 6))
 (segment (start 130.815031 105.515031) (end 130.815031 113.085031) (width 0.25) (layer B.Cu) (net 6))
 (segment (start 128.29 102.99) (end 130.815031 105.515031) (width 0.25) (layer B.Cu) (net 6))
 (segment (start 124.900001 106.379999) (end 125.75 105.53) (width 0.25) (layer B.Cu) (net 3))
 (segment (start 124.574999 106.705001) (end 124.900001 106.379999) (width 0.25) (layer B.Cu) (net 3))
 (segment (start 125.185999 111.785001) (end 124.574999 111.174001) (width 0.25) (layer B.Cu) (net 3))
 (segment (start 128.664003 111.785001) (end 125.185999 111.785001) (width 0.25) (layer B.Cu) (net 3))
 (segment (start 134.025 120.655) (end 129.465001 116.095001) (width 0.25) (layer B.Cu) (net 3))
 (segment (start 129.465001 112.585999) (end 128.664003 111.785001) (width 0.25) (layer B.Cu) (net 3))
 (segment (start 129.465001 116.095001) (end 129.465001 112.585999) (width 0.25) (layer B.Cu) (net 3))
 (segment (start 124.574999 111.174001) (end 124.574999 106.705001) (width 0.25) (layer B.Cu) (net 3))
 (segment (start 135.05 120.655) (end 134.025 120.655) (width 0.25) (layer B.Cu) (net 3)))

